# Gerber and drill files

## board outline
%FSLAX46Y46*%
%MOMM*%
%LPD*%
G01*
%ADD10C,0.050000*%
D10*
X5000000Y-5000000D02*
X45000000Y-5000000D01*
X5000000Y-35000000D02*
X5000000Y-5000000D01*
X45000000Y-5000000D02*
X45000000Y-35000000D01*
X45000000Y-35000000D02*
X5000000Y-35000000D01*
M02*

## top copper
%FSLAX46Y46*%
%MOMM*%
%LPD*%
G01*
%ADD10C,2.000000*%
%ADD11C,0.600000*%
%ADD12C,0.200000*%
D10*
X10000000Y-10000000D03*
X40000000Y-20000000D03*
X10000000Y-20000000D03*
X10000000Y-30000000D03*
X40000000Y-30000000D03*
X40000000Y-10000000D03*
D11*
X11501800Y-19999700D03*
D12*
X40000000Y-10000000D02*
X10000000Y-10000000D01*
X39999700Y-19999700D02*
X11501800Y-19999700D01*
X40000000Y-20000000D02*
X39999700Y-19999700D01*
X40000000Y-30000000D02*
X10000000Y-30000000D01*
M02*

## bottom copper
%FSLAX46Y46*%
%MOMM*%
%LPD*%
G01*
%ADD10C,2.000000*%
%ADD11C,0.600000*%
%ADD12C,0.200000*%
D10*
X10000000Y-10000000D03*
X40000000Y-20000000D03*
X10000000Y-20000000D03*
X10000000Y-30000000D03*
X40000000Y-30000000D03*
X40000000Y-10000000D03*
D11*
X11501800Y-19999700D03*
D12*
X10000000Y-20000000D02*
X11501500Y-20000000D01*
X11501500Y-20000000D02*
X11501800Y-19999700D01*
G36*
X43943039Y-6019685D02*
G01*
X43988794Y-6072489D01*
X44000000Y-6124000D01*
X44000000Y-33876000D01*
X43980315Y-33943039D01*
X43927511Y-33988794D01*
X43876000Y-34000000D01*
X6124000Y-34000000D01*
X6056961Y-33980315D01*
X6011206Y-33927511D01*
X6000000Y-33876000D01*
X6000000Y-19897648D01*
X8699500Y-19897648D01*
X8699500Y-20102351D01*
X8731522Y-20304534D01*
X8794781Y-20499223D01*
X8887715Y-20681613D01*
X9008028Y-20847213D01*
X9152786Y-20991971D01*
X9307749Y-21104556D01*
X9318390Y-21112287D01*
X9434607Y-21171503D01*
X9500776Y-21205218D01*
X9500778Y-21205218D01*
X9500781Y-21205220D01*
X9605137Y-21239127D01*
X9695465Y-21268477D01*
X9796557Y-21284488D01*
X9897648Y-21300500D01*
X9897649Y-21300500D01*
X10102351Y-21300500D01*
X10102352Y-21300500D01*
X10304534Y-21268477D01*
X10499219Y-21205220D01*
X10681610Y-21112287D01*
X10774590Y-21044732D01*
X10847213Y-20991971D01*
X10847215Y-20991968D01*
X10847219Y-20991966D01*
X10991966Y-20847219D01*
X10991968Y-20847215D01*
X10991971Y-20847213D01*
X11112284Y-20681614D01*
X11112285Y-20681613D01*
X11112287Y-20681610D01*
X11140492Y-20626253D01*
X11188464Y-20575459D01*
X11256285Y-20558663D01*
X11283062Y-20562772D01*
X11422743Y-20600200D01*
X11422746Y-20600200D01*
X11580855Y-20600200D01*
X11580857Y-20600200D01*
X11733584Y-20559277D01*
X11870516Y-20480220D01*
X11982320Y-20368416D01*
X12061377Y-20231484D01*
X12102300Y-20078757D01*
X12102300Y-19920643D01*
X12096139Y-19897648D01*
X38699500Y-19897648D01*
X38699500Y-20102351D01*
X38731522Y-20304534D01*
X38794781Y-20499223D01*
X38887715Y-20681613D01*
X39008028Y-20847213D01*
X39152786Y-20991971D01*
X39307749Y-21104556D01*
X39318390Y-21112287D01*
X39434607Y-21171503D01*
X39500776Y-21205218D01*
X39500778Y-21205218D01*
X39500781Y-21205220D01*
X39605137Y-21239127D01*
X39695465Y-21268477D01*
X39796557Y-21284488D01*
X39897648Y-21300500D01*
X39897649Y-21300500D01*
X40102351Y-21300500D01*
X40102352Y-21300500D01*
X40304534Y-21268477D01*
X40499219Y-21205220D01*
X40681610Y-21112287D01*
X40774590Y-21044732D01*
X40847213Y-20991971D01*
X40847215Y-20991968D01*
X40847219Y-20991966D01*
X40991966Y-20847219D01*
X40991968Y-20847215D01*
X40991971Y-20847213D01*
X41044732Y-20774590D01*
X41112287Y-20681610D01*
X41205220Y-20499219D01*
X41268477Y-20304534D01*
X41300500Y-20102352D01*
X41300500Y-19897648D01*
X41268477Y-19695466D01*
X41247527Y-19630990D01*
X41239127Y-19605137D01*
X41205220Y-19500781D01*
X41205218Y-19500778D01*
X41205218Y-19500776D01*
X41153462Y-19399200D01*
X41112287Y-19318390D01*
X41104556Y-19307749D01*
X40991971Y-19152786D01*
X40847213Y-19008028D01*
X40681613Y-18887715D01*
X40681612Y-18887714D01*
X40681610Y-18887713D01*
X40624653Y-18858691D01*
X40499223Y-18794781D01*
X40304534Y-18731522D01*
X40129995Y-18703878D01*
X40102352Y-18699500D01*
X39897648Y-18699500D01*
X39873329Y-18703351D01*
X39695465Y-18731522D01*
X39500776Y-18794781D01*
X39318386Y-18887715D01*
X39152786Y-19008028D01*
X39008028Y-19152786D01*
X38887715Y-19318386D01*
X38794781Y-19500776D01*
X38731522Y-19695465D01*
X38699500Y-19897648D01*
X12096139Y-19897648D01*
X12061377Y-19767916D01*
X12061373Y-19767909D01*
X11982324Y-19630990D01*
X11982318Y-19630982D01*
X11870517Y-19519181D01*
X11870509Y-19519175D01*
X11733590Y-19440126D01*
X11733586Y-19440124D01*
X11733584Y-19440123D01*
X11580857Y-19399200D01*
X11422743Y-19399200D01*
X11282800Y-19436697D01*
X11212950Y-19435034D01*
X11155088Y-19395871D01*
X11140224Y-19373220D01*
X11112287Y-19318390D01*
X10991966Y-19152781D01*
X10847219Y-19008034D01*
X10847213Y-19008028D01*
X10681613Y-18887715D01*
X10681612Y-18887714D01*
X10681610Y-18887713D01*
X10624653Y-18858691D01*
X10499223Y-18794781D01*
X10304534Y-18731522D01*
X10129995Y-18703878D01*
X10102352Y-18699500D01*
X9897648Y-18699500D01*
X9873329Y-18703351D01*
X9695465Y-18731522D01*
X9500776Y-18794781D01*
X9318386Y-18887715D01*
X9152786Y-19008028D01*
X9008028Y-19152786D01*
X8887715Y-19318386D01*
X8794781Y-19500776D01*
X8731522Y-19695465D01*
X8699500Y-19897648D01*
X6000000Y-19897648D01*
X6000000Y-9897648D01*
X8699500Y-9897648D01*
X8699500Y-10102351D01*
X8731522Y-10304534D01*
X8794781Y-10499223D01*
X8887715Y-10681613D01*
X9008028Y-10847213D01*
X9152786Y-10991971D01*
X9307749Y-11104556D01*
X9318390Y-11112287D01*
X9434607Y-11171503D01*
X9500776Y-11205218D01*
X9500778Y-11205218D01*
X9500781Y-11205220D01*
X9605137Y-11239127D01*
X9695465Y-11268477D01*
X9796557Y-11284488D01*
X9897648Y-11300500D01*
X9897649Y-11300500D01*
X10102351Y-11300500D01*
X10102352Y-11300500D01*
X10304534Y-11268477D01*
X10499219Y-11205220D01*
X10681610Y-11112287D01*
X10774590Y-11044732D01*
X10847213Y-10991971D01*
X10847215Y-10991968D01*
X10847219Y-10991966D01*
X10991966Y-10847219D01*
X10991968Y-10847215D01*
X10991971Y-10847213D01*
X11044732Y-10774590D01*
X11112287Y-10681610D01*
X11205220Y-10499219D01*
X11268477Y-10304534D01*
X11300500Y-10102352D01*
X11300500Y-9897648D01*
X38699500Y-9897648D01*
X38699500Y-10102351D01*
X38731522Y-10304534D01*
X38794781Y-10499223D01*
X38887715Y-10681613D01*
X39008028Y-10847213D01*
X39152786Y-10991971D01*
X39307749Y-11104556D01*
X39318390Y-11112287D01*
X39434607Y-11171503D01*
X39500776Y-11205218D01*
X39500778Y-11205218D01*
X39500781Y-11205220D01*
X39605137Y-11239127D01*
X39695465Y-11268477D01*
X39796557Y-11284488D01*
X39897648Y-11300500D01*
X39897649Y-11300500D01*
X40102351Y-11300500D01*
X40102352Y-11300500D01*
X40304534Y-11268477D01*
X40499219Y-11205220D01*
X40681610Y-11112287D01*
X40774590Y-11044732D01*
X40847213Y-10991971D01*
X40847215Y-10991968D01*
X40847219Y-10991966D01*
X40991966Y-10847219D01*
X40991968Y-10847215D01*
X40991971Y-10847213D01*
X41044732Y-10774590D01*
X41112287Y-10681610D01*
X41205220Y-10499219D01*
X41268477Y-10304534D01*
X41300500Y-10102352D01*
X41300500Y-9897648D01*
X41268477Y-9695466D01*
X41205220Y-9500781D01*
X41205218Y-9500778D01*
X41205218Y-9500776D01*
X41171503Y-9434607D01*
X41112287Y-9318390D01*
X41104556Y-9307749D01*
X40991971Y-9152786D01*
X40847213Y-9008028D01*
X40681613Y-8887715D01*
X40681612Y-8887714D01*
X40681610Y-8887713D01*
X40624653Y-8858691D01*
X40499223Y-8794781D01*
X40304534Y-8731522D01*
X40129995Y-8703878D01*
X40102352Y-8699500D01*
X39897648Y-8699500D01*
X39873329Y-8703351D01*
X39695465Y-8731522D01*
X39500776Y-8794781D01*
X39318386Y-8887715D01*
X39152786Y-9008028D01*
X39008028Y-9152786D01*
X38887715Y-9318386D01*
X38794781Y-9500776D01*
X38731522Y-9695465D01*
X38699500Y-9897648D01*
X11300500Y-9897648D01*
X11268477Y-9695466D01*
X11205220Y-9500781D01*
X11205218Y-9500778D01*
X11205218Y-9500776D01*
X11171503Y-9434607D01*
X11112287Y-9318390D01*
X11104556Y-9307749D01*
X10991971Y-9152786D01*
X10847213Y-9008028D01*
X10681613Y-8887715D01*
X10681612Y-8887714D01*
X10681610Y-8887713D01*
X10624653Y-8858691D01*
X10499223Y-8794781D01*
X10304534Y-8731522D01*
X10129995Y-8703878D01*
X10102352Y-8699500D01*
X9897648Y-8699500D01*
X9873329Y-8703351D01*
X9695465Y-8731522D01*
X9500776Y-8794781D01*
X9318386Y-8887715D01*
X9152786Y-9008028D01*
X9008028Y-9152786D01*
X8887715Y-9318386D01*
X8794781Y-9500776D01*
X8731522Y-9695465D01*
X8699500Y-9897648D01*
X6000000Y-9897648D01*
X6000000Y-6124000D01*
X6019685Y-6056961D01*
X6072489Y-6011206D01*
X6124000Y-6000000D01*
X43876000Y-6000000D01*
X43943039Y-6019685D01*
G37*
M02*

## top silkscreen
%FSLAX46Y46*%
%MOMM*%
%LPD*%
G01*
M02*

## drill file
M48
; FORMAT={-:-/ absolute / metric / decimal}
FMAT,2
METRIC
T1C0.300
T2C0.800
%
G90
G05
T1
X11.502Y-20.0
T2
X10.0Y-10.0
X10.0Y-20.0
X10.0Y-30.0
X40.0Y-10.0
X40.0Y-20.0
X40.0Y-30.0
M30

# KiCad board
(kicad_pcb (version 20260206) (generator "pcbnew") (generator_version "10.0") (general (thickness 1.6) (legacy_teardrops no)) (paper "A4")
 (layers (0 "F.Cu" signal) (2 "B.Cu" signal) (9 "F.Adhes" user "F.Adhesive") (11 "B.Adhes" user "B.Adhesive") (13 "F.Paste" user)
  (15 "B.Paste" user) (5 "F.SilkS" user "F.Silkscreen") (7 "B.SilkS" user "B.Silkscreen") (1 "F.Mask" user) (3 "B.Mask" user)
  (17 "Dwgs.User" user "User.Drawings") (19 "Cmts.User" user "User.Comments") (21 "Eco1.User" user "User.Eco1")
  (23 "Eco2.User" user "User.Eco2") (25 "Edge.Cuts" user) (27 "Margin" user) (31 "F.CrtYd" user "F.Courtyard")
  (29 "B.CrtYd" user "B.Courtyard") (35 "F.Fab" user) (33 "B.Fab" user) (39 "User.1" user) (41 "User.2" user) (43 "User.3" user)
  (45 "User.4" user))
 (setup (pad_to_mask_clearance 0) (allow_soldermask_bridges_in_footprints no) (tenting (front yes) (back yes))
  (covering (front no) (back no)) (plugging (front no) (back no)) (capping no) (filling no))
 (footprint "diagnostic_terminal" (layer "F.Cu") (at 10 10)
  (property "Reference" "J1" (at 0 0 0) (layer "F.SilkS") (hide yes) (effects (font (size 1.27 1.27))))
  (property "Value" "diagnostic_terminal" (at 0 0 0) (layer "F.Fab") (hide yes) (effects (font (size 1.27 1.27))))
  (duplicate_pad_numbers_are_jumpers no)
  (pad "1" thru_hole circle (at 0 0) (size 2 2) (drill 0.8) (layers "*.Cu") (remove_unused_layers no) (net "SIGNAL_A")))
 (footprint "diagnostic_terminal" (layer "F.Cu") (at 40 20)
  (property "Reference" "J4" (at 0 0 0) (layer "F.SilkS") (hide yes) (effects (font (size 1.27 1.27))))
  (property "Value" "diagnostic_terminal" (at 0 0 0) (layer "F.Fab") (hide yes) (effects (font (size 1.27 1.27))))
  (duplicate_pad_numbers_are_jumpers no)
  (pad "1" thru_hole circle (at 0 0) (size 2 2) (drill 0.8) (layers "*.Cu") (remove_unused_layers no) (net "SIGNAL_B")))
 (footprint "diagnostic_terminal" (layer "F.Cu") (at 10 20)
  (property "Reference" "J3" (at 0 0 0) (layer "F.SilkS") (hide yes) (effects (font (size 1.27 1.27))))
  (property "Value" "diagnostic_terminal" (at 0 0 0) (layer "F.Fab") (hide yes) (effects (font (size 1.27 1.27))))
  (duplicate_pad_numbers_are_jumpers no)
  (pad "1" thru_hole circle (at 0 0) (size 2 2) (drill 0.8) (layers "*.Cu") (remove_unused_layers no) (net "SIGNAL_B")))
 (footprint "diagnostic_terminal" (layer "F.Cu") (at 10 30)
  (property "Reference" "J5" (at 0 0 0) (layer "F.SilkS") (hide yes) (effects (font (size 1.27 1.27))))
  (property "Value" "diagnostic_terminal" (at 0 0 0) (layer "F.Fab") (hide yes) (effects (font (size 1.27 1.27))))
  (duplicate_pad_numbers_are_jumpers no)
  (pad "1" thru_hole circle (at 0 0) (size 2 2) (drill 0.8) (layers "*.Cu") (remove_unused_layers no) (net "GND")))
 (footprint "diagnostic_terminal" (layer "F.Cu") (at 40 30)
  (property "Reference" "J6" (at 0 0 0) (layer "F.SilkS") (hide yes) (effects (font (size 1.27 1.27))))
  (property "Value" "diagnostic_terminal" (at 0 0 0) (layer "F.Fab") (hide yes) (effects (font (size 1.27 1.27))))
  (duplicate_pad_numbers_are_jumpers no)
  (pad "1" thru_hole circle (at 0 0) (size 2 2) (drill 0.8) (layers "*.Cu") (remove_unused_layers no) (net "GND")))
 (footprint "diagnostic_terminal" (layer "F.Cu") (at 40 10)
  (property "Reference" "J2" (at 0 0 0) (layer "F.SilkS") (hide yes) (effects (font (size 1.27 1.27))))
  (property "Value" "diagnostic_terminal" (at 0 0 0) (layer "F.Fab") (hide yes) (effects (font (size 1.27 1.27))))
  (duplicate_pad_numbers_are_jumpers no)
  (pad "1" thru_hole circle (at 0 0) (size 2 2) (drill 0.8) (layers "*.Cu") (remove_unused_layers no) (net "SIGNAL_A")))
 (gr_line (start 5 5) (end 45 5) (stroke (width 0.05) (type default)) (layer "Edge.Cuts"))
 (gr_line (start 5 35) (end 5 5) (stroke (width 0.05) (type default)) (layer "Edge.Cuts"))
 (gr_line (start 45 5) (end 45 35) (stroke (width 0.05) (type default)) (layer "Edge.Cuts"))
 (gr_line (start 45 35) (end 5 35) (stroke (width 0.05) (type default)) (layer "Edge.Cuts"))
 (segment (start 40 10) (end 10 10) (width 0.2) (layer "F.Cu") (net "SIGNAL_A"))
 (segment (start 39.9997 19.9997) (end 11.5018 19.9997) (width 0.2) (layer "F.Cu") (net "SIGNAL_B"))
 (segment (start 40 20) (end 39.9997 19.9997) (width 0.2) (layer "F.Cu") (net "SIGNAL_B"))
 (via (at 11.5018 19.9997) (size 0.6) (drill 0.3) (layers "F.Cu" "B.Cu") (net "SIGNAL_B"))
 (segment (start 10 20) (end 11.5015 20) (width 0.2) (layer "B.Cu") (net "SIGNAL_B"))
 (segment (start 11.5015 20) (end 11.5018 19.9997) (width 0.2) (layer "B.Cu") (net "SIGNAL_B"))
 (segment (start 40 30) (end 10 30) (width 0.2) (layer "F.Cu") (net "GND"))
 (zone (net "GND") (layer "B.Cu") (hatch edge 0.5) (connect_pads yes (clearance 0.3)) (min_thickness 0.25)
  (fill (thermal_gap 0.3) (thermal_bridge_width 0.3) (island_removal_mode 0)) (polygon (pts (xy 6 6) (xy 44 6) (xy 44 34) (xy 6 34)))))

